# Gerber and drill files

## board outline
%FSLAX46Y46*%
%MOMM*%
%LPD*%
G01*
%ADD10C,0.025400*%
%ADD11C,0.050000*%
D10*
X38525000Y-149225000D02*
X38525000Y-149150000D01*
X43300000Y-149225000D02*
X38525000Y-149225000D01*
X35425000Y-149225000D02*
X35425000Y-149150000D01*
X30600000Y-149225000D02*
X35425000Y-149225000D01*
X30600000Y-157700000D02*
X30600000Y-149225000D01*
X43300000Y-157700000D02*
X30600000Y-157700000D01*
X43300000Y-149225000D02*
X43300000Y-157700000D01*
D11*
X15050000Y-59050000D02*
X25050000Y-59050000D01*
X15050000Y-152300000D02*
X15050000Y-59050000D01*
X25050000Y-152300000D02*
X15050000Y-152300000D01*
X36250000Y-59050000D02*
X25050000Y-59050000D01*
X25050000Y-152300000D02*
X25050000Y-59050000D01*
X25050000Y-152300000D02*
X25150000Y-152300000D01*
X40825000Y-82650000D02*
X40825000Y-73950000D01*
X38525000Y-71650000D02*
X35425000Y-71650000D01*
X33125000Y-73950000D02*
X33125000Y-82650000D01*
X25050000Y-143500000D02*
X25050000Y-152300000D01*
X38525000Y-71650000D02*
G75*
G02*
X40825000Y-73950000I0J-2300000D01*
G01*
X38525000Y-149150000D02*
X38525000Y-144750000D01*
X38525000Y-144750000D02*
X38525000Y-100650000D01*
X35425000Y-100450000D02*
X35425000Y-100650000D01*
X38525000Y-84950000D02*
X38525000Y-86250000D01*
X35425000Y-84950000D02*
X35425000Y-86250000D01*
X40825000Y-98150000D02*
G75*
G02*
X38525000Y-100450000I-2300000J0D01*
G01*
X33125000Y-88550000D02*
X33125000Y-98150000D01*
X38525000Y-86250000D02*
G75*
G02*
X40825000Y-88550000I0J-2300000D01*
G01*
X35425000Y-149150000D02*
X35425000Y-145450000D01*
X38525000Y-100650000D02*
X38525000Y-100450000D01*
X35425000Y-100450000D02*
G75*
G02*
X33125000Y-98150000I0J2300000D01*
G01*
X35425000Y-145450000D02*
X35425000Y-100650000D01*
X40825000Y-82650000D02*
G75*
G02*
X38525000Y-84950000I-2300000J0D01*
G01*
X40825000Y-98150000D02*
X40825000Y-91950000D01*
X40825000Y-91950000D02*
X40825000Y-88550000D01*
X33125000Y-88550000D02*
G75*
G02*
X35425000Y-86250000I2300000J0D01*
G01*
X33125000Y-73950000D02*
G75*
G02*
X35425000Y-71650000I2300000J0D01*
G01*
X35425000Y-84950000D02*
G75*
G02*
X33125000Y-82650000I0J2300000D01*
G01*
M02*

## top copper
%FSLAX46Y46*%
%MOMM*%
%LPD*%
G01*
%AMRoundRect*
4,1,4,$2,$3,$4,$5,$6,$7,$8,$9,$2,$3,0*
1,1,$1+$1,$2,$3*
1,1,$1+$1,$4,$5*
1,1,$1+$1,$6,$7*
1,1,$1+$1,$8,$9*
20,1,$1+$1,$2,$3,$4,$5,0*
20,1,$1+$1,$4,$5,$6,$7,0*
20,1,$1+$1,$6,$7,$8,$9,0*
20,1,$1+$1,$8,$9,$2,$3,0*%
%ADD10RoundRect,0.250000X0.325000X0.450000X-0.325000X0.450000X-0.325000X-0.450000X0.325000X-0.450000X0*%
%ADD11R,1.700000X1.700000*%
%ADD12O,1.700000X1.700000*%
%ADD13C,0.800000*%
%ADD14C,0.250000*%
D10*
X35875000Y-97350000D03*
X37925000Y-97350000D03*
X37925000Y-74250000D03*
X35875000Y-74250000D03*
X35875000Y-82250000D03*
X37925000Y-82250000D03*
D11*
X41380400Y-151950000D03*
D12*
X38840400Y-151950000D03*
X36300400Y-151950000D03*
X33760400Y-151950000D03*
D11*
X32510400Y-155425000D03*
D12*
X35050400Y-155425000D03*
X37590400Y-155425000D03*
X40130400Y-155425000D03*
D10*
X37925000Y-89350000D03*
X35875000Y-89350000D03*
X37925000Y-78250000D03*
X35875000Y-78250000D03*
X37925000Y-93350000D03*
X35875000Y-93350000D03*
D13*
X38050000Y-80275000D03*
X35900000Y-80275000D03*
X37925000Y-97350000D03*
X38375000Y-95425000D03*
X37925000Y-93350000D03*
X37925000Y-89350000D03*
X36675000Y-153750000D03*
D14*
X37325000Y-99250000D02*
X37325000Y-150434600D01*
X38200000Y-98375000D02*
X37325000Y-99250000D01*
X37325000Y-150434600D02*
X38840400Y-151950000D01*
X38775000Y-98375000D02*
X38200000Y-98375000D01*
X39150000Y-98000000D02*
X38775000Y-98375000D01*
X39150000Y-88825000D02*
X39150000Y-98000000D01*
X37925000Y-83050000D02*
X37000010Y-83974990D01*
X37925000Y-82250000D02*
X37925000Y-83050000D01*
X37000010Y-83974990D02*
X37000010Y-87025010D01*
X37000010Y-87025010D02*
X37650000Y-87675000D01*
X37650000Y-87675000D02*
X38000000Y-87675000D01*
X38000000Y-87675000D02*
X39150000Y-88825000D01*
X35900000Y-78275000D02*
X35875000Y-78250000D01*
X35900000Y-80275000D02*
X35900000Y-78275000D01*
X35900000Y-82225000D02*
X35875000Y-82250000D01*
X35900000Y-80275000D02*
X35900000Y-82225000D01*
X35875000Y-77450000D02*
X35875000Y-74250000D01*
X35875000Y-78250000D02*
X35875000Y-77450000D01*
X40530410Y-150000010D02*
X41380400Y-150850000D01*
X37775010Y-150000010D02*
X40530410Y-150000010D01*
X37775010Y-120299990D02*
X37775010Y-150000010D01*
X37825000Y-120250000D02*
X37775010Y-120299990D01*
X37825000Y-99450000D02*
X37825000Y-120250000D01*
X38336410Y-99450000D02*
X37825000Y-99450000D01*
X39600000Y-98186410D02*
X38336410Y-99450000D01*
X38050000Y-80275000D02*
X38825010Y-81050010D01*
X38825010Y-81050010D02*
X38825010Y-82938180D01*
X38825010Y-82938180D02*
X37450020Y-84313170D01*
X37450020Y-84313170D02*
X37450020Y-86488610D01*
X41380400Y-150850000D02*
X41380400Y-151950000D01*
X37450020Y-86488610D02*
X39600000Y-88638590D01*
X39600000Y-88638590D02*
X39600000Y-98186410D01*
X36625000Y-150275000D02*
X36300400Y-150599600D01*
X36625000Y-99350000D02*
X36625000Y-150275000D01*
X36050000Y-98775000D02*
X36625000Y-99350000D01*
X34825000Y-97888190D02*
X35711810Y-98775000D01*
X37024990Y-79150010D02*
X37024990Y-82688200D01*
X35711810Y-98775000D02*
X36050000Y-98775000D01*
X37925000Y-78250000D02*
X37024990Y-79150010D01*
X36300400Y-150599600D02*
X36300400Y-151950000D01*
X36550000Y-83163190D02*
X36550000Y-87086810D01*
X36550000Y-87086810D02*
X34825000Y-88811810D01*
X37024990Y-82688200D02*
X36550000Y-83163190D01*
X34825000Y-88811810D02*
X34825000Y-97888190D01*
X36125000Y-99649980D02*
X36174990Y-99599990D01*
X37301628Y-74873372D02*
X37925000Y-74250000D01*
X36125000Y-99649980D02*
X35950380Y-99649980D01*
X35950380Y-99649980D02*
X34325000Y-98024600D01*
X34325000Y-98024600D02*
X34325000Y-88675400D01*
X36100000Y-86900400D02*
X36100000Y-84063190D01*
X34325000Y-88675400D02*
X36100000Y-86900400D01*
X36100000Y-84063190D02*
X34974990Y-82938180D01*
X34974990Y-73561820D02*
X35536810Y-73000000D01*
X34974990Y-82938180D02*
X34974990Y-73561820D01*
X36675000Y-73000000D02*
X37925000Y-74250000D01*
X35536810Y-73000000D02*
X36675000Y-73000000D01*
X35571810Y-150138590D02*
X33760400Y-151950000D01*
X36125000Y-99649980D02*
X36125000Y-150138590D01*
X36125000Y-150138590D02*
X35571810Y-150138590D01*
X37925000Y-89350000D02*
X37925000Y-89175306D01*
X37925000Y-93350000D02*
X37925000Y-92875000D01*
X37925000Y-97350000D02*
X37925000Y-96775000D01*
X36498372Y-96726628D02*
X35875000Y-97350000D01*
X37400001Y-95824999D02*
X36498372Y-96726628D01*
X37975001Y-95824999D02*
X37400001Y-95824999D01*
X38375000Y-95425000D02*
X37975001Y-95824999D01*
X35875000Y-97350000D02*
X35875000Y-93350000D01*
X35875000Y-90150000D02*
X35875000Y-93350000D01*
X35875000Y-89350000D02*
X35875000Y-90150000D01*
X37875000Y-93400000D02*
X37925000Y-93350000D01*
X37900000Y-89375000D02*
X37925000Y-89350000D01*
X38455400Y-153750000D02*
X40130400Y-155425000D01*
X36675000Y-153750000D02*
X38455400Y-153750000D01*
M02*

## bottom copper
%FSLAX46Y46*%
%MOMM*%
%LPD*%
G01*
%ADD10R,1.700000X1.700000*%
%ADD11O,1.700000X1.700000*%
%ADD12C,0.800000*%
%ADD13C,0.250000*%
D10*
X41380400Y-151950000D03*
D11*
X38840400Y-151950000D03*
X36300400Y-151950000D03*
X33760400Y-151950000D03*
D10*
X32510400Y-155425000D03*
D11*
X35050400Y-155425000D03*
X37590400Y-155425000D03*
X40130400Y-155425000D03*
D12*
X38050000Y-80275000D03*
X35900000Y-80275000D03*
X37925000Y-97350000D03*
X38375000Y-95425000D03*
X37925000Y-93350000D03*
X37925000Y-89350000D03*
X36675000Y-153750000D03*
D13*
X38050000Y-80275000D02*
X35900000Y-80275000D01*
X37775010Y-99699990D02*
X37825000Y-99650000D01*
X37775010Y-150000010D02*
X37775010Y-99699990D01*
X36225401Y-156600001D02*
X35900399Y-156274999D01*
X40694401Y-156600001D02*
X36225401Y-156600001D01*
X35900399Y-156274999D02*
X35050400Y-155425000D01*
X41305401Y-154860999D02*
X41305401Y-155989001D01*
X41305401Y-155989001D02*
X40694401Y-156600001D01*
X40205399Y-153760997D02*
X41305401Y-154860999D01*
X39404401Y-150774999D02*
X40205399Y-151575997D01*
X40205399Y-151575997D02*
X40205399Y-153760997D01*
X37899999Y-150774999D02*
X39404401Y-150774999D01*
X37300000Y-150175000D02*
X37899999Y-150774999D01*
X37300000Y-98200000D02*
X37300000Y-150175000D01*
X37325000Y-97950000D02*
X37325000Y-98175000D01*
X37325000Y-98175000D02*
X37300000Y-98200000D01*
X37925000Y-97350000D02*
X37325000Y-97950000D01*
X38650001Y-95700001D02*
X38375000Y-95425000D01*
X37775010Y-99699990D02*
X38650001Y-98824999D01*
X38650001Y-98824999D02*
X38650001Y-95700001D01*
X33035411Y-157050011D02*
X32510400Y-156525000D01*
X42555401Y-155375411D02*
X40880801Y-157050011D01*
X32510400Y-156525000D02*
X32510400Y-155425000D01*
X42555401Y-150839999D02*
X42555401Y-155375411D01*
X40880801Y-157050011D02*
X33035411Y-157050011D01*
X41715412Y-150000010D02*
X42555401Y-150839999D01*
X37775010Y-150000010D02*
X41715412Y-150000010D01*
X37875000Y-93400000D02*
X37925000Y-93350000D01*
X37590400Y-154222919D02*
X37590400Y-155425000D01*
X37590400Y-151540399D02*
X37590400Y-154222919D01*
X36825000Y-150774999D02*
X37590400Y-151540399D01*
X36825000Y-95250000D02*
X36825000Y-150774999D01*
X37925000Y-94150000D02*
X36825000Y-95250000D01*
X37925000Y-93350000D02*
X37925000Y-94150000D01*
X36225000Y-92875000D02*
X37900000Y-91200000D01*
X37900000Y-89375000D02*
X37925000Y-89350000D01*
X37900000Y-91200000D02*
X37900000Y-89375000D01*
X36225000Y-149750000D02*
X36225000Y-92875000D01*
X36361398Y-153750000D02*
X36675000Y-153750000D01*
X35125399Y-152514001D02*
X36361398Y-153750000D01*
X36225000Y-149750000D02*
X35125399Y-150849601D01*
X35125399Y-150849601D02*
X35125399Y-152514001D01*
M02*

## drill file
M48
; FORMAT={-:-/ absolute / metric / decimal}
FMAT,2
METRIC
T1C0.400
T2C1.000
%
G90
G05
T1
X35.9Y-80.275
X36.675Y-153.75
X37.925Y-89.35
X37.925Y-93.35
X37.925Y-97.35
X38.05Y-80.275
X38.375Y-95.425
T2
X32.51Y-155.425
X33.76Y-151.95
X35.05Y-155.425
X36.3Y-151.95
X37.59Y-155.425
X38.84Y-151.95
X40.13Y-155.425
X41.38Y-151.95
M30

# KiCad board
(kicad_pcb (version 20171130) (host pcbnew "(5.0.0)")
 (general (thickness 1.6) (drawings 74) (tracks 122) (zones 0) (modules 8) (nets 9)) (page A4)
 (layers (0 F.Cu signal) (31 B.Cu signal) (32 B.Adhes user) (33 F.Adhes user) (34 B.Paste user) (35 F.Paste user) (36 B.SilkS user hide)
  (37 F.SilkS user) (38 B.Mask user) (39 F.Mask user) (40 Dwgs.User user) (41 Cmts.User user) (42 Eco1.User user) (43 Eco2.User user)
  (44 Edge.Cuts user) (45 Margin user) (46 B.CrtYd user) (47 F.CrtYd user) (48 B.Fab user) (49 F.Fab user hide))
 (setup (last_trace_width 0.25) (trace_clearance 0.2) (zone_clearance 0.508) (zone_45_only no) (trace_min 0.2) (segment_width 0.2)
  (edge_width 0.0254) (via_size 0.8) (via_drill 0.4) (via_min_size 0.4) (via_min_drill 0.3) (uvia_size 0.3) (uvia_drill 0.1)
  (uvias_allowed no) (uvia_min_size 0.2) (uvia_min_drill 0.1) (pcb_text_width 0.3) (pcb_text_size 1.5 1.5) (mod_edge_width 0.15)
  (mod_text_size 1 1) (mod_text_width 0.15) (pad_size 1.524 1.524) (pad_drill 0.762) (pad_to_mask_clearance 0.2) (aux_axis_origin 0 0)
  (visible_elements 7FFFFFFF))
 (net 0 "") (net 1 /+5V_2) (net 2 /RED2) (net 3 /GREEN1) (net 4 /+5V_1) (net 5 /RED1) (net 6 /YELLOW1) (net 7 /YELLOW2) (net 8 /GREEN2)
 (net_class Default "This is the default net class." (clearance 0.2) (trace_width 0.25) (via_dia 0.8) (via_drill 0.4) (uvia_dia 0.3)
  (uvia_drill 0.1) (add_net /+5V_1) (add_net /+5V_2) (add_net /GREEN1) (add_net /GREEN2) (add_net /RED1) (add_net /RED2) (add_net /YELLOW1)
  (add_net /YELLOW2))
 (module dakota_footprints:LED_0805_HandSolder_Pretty (layer F.Cu) (at 36.9 97.35 180)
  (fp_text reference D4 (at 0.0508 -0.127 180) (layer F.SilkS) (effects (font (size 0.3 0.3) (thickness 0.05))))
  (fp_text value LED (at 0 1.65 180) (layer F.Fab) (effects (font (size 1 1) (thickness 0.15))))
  (pad 2 smd roundrect (at 1.025 0 180) (size 1.15 1.4) (layers F.Cu F.Paste F.Mask) (roundrect_rratio 0.217391) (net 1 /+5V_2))
  (pad 1 smd roundrect (at -1.025 0 180) (size 1.15 1.4) (layers F.Cu F.Paste F.Mask) (roundrect_rratio 0.217391) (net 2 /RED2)))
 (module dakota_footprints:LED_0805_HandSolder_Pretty (layer F.Cu) (at 36.9 74.25 180)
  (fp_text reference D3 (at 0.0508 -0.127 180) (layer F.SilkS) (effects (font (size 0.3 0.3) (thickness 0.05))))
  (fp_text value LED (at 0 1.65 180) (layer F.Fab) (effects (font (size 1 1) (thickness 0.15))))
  (pad 1 smd roundrect (at -1.025 0 180) (size 1.15 1.4) (layers F.Cu F.Paste F.Mask) (roundrect_rratio 0.217391) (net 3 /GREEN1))
  (pad 2 smd roundrect (at 1.025 0 180) (size 1.15 1.4) (layers F.Cu F.Paste F.Mask) (roundrect_rratio 0.217391) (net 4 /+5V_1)))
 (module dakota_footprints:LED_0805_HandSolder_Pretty (layer F.Cu) (at 36.9 82.25 180)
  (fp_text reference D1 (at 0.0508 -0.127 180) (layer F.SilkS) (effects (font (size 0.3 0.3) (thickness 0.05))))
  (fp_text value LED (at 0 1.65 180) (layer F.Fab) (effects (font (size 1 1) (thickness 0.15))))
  (pad 2 smd roundrect (at 1.025 0 180) (size 1.15 1.4) (layers F.Cu F.Paste F.Mask) (roundrect_rratio 0.217391) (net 4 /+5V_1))
  (pad 1 smd roundrect (at -1.025 0 180) (size 1.15 1.4) (layers F.Cu F.Paste F.Mask) (roundrect_rratio 0.217391) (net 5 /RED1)))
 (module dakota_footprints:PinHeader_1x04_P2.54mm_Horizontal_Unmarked (layer F.Cu) (at 41.3804 151.95 270)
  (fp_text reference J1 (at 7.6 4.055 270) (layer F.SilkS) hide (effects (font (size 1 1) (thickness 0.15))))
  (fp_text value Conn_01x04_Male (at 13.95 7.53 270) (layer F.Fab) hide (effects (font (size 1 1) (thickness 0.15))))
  (pad 1 thru_hole rect (at 0 0 270) (size 1.7 1.7) (drill 1) (layers *.Cu *.Mask) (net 4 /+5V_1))
  (pad 2 thru_hole oval (at 0 2.54 270) (size 1.7 1.7) (drill 1) (layers *.Cu *.Mask) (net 5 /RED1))
  (pad 3 thru_hole oval (at 0 5.08 270) (size 1.7 1.7) (drill 1) (layers *.Cu *.Mask) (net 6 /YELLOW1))
  (pad 4 thru_hole oval (at 0 7.62 270) (size 1.7 1.7) (drill 1) (layers *.Cu *.Mask) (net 3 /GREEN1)))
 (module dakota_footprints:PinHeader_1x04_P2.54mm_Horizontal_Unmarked (layer B.Cu) (at 32.5104 155.425 270)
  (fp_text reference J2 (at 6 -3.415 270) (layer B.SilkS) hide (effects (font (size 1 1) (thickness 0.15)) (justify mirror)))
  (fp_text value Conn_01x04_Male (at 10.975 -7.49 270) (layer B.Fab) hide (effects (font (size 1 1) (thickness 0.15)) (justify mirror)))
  (pad 1 thru_hole rect (at 0 0 270) (size 1.7 1.7) (drill 1) (layers *.Cu *.Mask) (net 1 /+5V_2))
  (pad 2 thru_hole oval (at 0 -2.54 270) (size 1.7 1.7) (drill 1) (layers *.Cu *.Mask) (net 2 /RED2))
  (pad 3 thru_hole oval (at 0 -5.08 270) (size 1.7 1.7) (drill 1) (layers *.Cu *.Mask) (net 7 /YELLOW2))
  (pad 4 thru_hole oval (at 0 -7.62 270) (size 1.7 1.7) (drill 1) (layers *.Cu *.Mask) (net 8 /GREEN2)))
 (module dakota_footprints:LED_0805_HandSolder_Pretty (layer F.Cu) (at 36.9 89.35 180)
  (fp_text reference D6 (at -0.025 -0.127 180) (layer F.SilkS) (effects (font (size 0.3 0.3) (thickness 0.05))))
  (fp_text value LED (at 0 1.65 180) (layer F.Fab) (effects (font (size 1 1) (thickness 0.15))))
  (pad 1 smd roundrect (at -1.025 0 180) (size 1.15 1.4) (layers F.Cu F.Paste F.Mask) (roundrect_rratio 0.217391) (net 8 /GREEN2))
  (pad 2 smd roundrect (at 1.025 0 180) (size 1.15 1.4) (layers F.Cu F.Paste F.Mask) (roundrect_rratio 0.217391) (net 1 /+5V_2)))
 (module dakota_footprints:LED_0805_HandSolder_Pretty (layer F.Cu) (at 36.9 78.25 180)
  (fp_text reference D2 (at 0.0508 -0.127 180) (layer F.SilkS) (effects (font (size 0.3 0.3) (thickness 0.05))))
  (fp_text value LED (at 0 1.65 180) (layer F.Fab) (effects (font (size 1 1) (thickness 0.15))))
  (pad 1 smd roundrect (at -1.025 0 180) (size 1.15 1.4) (layers F.Cu F.Paste F.Mask) (roundrect_rratio 0.217391) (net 6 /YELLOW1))
  (pad 2 smd roundrect (at 1.025 0 180) (size 1.15 1.4) (layers F.Cu F.Paste F.Mask) (roundrect_rratio 0.217391) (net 4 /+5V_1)))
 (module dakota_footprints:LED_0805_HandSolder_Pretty (layer F.Cu) (at 36.9 93.35 180)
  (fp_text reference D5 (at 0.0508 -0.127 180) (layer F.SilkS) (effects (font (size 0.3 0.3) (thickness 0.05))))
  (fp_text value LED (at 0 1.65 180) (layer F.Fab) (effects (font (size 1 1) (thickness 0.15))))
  (pad 1 smd roundrect (at -1.025 0 180) (size 1.15 1.4) (layers F.Cu F.Paste F.Mask) (roundrect_rratio 0.217391) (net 7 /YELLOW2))
  (pad 2 smd roundrect (at 1.025 0 180) (size 1.15 1.4) (layers F.Cu F.Paste F.Mask) (roundrect_rratio 0.217391) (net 1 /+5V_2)))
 (gr_line (start 38.525 149.225) (end 38.525 149.15) (layer Edge.Cuts) (width 0.0254))
 (gr_line (start 43.3 149.225) (end 38.525 149.225) (layer Edge.Cuts) (width 0.0254))
 (gr_line (start 35.425 149.225) (end 35.425 149.15) (layer Edge.Cuts) (width 0.0254))
 (gr_line (start 30.6 149.225) (end 35.425 149.225) (layer Edge.Cuts) (width 0.0254))
 (gr_line (start 30.6 157.7) (end 30.6 149.225) (layer Edge.Cuts) (width 0.0254))
 (gr_line (start 43.3 157.7) (end 30.6 157.7) (layer Edge.Cuts) (width 0.0254))
 (gr_line (start 43.3 149.225) (end 43.3 157.7) (layer Edge.Cuts) (width 0.0254))
 (gr_line (start 15.05 59.05) (end 25.05 59.05) (layer Edge.Cuts) (width 0.05))
 (gr_line (start 15.05 152.3) (end 15.05 59.05) (layer Edge.Cuts) (width 0.05))
 (gr_line (start 25.05 152.3) (end 15.05 152.3) (layer Edge.Cuts) (width 0.05))
 (gr_line (start 36.25 59.05) (end 25.05 59.05) (layer Edge.Cuts) (width 0.05))
 (gr_line (start 25.05 152.3) (end 25.05 59.05) (layer Edge.Cuts) (width 0.05))
 (gr_line (start 25.05 152.3) (end 25.15 152.3) (layer Edge.Cuts) (width 0.05))
 (gr_line (start 40.825 82.65) (end 40.825 73.95) (layer Edge.Cuts) (width 0.05))
 (gr_line (start 38.525 71.65) (end 35.425 71.65) (layer Edge.Cuts) (width 0.05))
 (gr_line (start 33.125 73.95) (end 33.125 82.65) (layer Edge.Cuts) (width 0.05))
 (gr_line (start 25.05 143.5) (end 25.05 152.3) (layer Edge.Cuts) (width 0.05))
 (gr_arc (start 38.525 73.95) (end 40.825 73.95) (angle -90) (layer Edge.Cuts) (width 0.05))
 (gr_line (start 38.525 149.15) (end 38.525 144.75) (layer Edge.Cuts) (width 0.05))
 (gr_line (start 38.525 144.75) (end 38.525 100.65) (layer Edge.Cuts) (width 0.05))
 (gr_line (start 35.425 100.45) (end 35.425 100.65) (layer Edge.Cuts) (width 0.05))
 (gr_line (start 38.525 84.95) (end 38.525 86.25) (layer Edge.Cuts) (width 0.05))
 (gr_line (start 35.425 84.95) (end 35.425 86.25) (layer Edge.Cuts) (width 0.05))
 (gr_arc (start 38.525 98.15) (end 38.525 100.45) (angle -90) (layer Edge.Cuts) (width 0.05))
 (gr_line (start 33.125 88.55) (end 33.125 98.15) (layer Edge.Cuts) (width 0.05))
 (gr_arc (start 38.525 88.55) (end 40.825 88.55) (angle -90) (layer Edge.Cuts) (width 0.05))
 (gr_line (start 35.425 149.15) (end 35.425 145.45) (layer Edge.Cuts) (width 0.05))
 (gr_line (start 38.525 100.65) (end 38.525 100.45) (layer Edge.Cuts) (width 0.05))
 (gr_arc (start 35.425 98.15) (end 33.125 98.15) (angle -90) (layer Edge.Cuts) (width 0.05))
 (gr_line (start 35.425 145.45) (end 35.425 100.65) (layer Edge.Cuts) (width 0.05))
 (gr_arc (start 38.525 82.65) (end 38.525 84.95) (angle -90) (layer Edge.Cuts) (width 0.05))
 (gr_line (start 40.825 98.15) (end 40.825 91.95) (layer Edge.Cuts) (width 0.05))
 (gr_line (start 40.825 91.95) (end 40.825 88.55) (layer Edge.Cuts) (width 0.05))
 (gr_arc (start 35.425 88.55) (end 35.425 86.25) (angle -90) (layer Edge.Cuts) (width 0.05))
 (gr_arc (start 35.425 73.95) (end 35.425 71.65) (angle -90) (layer Edge.Cuts) (width 0.05))
 (gr_arc (start 35.425 82.65) (end 33.125 82.65) (angle -90) (layer Edge.Cuts) (width 0.05))
 (segment (start 37.325 99.25) (end 37.325 150.4346) (width 0.25) (layer F.Cu) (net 5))
 (segment (start 38.2 98.375) (end 37.325 99.25) (width 0.25) (layer F.Cu) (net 5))
 (segment (start 37.325 150.4346) (end 38.8404 151.95) (width 0.25) (layer F.Cu) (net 5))
 (segment (start 38.775 98.375) (end 38.2 98.375) (width 0.25) (layer F.Cu) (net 5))
 (segment (start 39.15 98) (end 38.775 98.375) (width 0.25) (layer F.Cu) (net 5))
 (segment (start 39.15 88.825) (end 39.15 98) (width 0.25) (layer F.Cu) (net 5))
 (segment (start 37.925 83.05) (end 37.00001 83.97499) (width 0.25) (layer F.Cu) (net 5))
 (segment (start 37.925 82.25) (end 37.925 83.05) (width 0.25) (layer F.Cu) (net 5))
 (segment (start 37.00001 83.97499) (end 37.00001 87.02501) (width 0.25) (layer F.Cu) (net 5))
 (segment (start 37.00001 87.02501) (end 37.65 87.675) (width 0.25) (layer F.Cu) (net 5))
 (segment (start 37.65 87.675) (end 38 87.675) (width 0.25) (layer F.Cu) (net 5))
 (segment (start 38 87.675) (end 39.15 88.825) (width 0.25) (layer F.Cu) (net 5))
 (via (at 38.05 80.275) (size 0.8) (drill 0.4) (layers F.Cu B.Cu) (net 4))
 (via (at 35.9 80.275) (size 0.8) (drill 0.4) (layers F.Cu B.Cu) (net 4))
 (segment (start 38.05 80.275) (end 35.9 80.275) (width 0.25) (layer B.Cu) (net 4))
 (segment (start 35.9 78.275) (end 35.875 78.25) (width 0.25) (layer F.Cu) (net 4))
 (segment (start 35.9 80.275) (end 35.9 78.275) (width 0.25) (layer F.Cu) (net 4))
 (segment (start 35.9 82.225) (end 35.875 82.25) (width 0.25) (layer F.Cu) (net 4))
 (segment (start 35.9 80.275) (end 35.9 82.225) (width 0.25) (layer F.Cu) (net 4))
 (segment (start 35.875 77.45) (end 35.875 74.25) (width 0.25) (layer F.Cu) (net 4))
 (segment (start 35.875 78.25) (end 35.875 77.45) (width 0.25) (layer F.Cu) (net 4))
 (segment (start 40.53041 150.00001) (end 41.3804 150.85) (width 0.25) (layer F.Cu) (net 4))
 (segment (start 37.77501 150.00001) (end 40.53041 150.00001) (width 0.25) (layer F.Cu) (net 4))
 (segment (start 37.77501 120.29999) (end 37.77501 150.00001) (width 0.25) (layer F.Cu) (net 4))
 (segment (start 37.825 120.25) (end 37.77501 120.29999) (width 0.25) (layer F.Cu) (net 4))
 (segment (start 37.825 99.45) (end 37.825 120.25) (width 0.25) (layer F.Cu) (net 4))
 (segment (start 38.33641 99.45) (end 37.825 99.45) (width 0.25) (layer F.Cu) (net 4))
 (segment (start 39.6 98.18641) (end 38.33641 99.45) (width 0.25) (layer F.Cu) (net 4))
 (segment (start 38.05 80.275) (end 38.82501 81.05001) (width 0.25) (layer F.Cu) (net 4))
 (segment (start 38.82501 81.05001) (end 38.82501 82.93818) (width 0.25) (layer F.Cu) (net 4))
 (segment (start 38.82501 82.93818) (end 37.45002 84.31317) (width 0.25) (layer F.Cu) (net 4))
 (segment (start 37.45002 84.31317) (end 37.45002 86.48861) (width 0.25) (layer F.Cu) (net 4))
 (segment (start 41.3804 150.85) (end 41.3804 151.95) (width 0.25) (layer F.Cu) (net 4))
 (segment (start 37.45002 86.48861) (end 39.6 88.63859) (width 0.25) (layer F.Cu) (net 4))
 (segment (start 39.6 88.63859) (end 39.6 98.18641) (width 0.25) (layer F.Cu) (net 4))
 (segment (start 36.625 150.275) (end 36.3004 150.5996) (width 0.25) (layer F.Cu) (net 6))
 (segment (start 36.625 99.35) (end 36.625 150.275) (width 0.25) (layer F.Cu) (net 6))
 (segment (start 36.05 98.775) (end 36.625 99.35) (width 0.25) (layer F.Cu) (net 6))
 (segment (start 34.825 97.88819) (end 35.71181 98.775) (width 0.25) (layer F.Cu) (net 6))
 (segment (start 37.02499 79.15001) (end 37.02499 82.6882) (width 0.25) (layer F.Cu) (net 6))
 (segment (start 35.71181 98.775) (end 36.05 98.775) (width 0.25) (layer F.Cu) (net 6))
 (segment (start 37.925 78.25) (end 37.02499 79.15001) (width 0.25) (layer F.Cu) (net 6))
 (segment (start 36.3004 150.5996) (end 36.3004 151.95) (width 0.25) (layer F.Cu) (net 6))
 (segment (start 36.55 83.16319) (end 36.55 87.08681) (width 0.25) (layer F.Cu) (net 6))
 (segment (start 36.55 87.08681) (end 34.825 88.81181) (width 0.25) (layer F.Cu) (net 6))
 (segment (start 37.02499 82.6882) (end 36.55 83.16319) (width 0.25) (layer F.Cu) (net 6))
 (segment (start 34.825 88.81181) (end 34.825 97.88819) (width 0.25) (layer F.Cu) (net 6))
 (segment (start 36.125 99.64998) (end 36.17499 99.59999) (width 0.25) (layer F.Cu) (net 3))
 (segment (start 37.301628 74.873372) (end 37.925 74.25) (width 0.25) (layer F.Cu) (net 3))
 (segment (start 36.125 99.64998) (end 35.95038 99.64998) (width 0.25) (layer F.Cu) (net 3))
 (segment (start 35.95038 99.64998) (end 34.325 98.0246) (width 0.25) (layer F.Cu) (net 3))
 (segment (start 34.325 98.0246) (end 34.325 88.6754) (width 0.25) (layer F.Cu) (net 3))
 (segment (start 36.1 86.9004) (end 36.1 84.06319) (width 0.25) (layer F.Cu) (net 3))
 (segment (start 34.325 88.6754) (end 36.1 86.9004) (width 0.25) (layer F.Cu) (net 3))
 (segment (start 36.1 84.06319) (end 34.97499 82.93818) (width 0.25) (layer F.Cu) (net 3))
 (segment (start 34.97499 73.56182) (end 35.53681 73) (width 0.25) (layer F.Cu) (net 3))
 (segment (start 34.97499 82.93818) (end 34.97499 73.56182) (width 0.25) (layer F.Cu) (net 3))
 (segment (start 36.675 73) (end 37.925 74.25) (width 0.25) (layer F.Cu) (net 3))
 (segment (start 35.53681 73) (end 36.675 73) (width 0.25) (layer F.Cu) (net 3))
 (segment (start 35.57181 150.13859) (end 33.7604 151.95) (width 0.25) (layer F.Cu) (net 3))
 (segment (start 36.125 99.64998) (end 36.125 150.13859) (width 0.25) (layer F.Cu) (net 3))
 (segment (start 36.125 150.13859) (end 35.57181 150.13859) (width 0.25) (layer F.Cu) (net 3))
 (segment (start 37.925 89.35) (end 37.925 89.175306) (width 0.25) (layer F.Cu) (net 8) (status 30))
 (segment (start 37.77501 99.69999) (end 37.825 99.65) (width 0.25) (layer B.Cu) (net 1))
 (segment (start 37.77501 150.00001) (end 37.77501 99.69999) (width 0.25) (layer B.Cu) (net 1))
 (segment (start 37.925 93.35) (end 37.925 92.875) (width 0.25) (layer F.Cu) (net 7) (status 30))
 (segment (start 37.925 97.35) (end 37.925 96.775) (width 0.25) (layer F.Cu) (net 2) (status 30))
 (via (at 37.925 97.35) (size 0.8) (drill 0.4) (layers F.Cu B.Cu) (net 2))
 (segment (start 36.225401 156.600001) (end 35.900399 156.274999) (width 0.25) (layer B.Cu) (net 2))
 (segment (start 40.694401 156.600001) (end 36.225401 156.600001) (width 0.25) (layer B.Cu) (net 2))
 (segment (start 35.900399 156.274999) (end 35.0504 155.425) (width 0.25) (layer B.Cu) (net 2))
 (segment (start 41.305401 154.860999) (end 41.305401 155.989001) (width 0.25) (layer B.Cu) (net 2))
 (segment (start 41.305401 155.989001) (end 40.694401 156.600001) (width 0.25) (layer B.Cu) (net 2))
 (segment (start 40.205399 153.760997) (end 41.305401 154.860999) (width 0.25) (layer B.Cu) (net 2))
 (segment (start 39.404401 150.774999) (end 40.205399 151.575997) (width 0.25) (layer B.Cu) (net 2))
 (segment (start 40.205399 151.575997) (end 40.205399 153.760997) (width 0.25) (layer B.Cu) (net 2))
 (segment (start 37.899999 150.774999) (end 39.404401 150.774999) (width 0.25) (layer B.Cu) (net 2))
 (segment (start 37.3 150.175) (end 37.899999 150.774999) (width 0.25) (layer B.Cu) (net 2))
 (segment (start 37.3 98.2) (end 37.3 150.175) (width 0.25) (layer B.Cu) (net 2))
 (segment (start 37.325 97.95) (end 37.325 98.175) (width 0.25) (layer B.Cu) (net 2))
 (segment (start 37.325 98.175) (end 37.3 98.2) (width 0.25) (layer B.Cu) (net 2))
 (segment (start 37.925 97.35) (end 37.325 97.95) (width 0.25) (layer B.Cu) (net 2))
 (via (at 38.375 95.425) (size 0.8) (drill 0.4) (layers F.Cu B.Cu) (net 1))
 (segment (start 38.650001 95.700001) (end 38.375 95.425) (width 0.25) (layer B.Cu) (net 1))
 (segment (start 37.77501 99.69999) (end 38.650001 98.824999) (width 0.25) (layer B.Cu) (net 1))
 (segment (start 38.650001 98.824999) (end 38.650001 95.700001) (width 0.25) (layer B.Cu) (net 1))
 (segment (start 36.498372 96.726628) (end 35.875 97.35) (width 0.25) (layer F.Cu) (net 1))
 (segment (start 37.400001 95.824999) (end 36.498372 96.726628) (width 0.25) (layer F.Cu) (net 1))
 (segment (start 37.975001 95.824999) (end 37.400001 95.824999) (width 0.25) (layer F.Cu) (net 1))
 (segment (start 38.375 95.425) (end 37.975001 95.824999) (width 0.25) (layer F.Cu) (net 1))
 (segment (start 35.875 97.35) (end 35.875 93.35) (width 0.25) (layer F.Cu) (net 1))
 (segment (start 35.875 90.15) (end 35.875 93.35) (width 0.25) (layer F.Cu) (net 1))
 (segment (start 35.875 89.35) (end 35.875 90.15) (width 0.25) (layer F.Cu) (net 1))
 (segment (start 33.035411 157.050011) (end 32.5104 156.525) (width 0.25) (layer B.Cu) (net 1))
 (segment (start 42.555401 155.375411) (end 40.880801 157.050011) (width 0.25) (layer B.Cu) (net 1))
 (segment (start 32.5104 156.525) (end 32.5104 155.425) (width 0.25) (layer B.Cu) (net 1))
 (segment (start 42.555401 150.839999) (end 42.555401 155.375411) (width 0.25) (layer B.Cu) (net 1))
 (segment (start 40.880801 157.050011) (end 33.035411 157.050011) (width 0.25) (layer B.Cu) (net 1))
 (segment (start 41.715412 150.00001) (end 42.555401 150.839999) (width 0.25) (layer B.Cu) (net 1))
 (segment (start 37.77501 150.00001) (end 41.715412 150.00001) (width 0.25) (layer B.Cu) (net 1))
 (segment (start 37.875 93.4) (end 37.925 93.35) (width 0.25) (layer F.Cu) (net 7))
 (segment (start 37.875 93.4) (end 37.925 93.35) (width 0.25) (layer B.Cu) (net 7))
 (via (at 37.925 93.35) (size 0.8) (drill 0.4) (layers F.Cu B.Cu) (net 7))
 (segment (start 37.5904 154.222919) (end 37.5904 155.425) (width 0.25) (layer B.Cu) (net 7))
 (segment (start 37.5904 151.540399) (end 37.5904 154.222919) (width 0.25) (layer B.Cu) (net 7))
 (segment (start 36.825 150.774999) (end 37.5904 151.540399) (width 0.25) (layer B.Cu) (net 7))
 (segment (start 36.825 95.25) (end 36.825 150.774999) (width 0.25) (layer B.Cu) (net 7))
 (segment (start 37.925 94.15) (end 36.825 95.25) (width 0.25) (layer B.Cu) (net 7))
 (segment (start 37.925 93.35) (end 37.925 94.15) (width 0.25) (layer B.Cu) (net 7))
 (segment (start 37.9 89.375) (end 37.925 89.35) (width 0.25) (layer F.Cu) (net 8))
 (segment (start 36.225 92.875) (end 37.9 91.2) (width 0.25) (layer B.Cu) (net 8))
 (segment (start 37.9 89.375) (end 37.925 89.35) (width 0.25) (layer B.Cu) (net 8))
 (segment (start 37.9 91.2) (end 37.9 89.375) (width 0.25) (layer B.Cu) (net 8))
 (via (at 37.925 89.35) (size 0.8) (drill 0.4) (layers F.Cu B.Cu) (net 8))
 (segment (start 36.225 149.75) (end 36.225 92.875) (width 0.25) (layer B.Cu) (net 8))
 (via (at 36.675 153.75) (size 0.8) (drill 0.4) (layers F.Cu B.Cu) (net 8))
 (segment (start 36.361398 153.75) (end 36.675 153.75) (width 0.25) (layer B.Cu) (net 8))
 (segment (start 35.125399 152.514001) (end 36.361398 153.75) (width 0.25) (layer B.Cu) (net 8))
 (segment (start 36.225 149.75) (end 35.125399 150.849601) (width 0.25) (layer B.Cu) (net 8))
 (segment (start 35.125399 150.849601) (end 35.125399 152.514001) (width 0.25) (layer B.Cu) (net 8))
 (segment (start 38.4554 153.75) (end 40.1304 155.425) (width 0.25) (layer F.Cu) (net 8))
 (segment (start 36.675 153.75) (end 38.4554 153.75) (width 0.25) (layer F.Cu) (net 8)))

